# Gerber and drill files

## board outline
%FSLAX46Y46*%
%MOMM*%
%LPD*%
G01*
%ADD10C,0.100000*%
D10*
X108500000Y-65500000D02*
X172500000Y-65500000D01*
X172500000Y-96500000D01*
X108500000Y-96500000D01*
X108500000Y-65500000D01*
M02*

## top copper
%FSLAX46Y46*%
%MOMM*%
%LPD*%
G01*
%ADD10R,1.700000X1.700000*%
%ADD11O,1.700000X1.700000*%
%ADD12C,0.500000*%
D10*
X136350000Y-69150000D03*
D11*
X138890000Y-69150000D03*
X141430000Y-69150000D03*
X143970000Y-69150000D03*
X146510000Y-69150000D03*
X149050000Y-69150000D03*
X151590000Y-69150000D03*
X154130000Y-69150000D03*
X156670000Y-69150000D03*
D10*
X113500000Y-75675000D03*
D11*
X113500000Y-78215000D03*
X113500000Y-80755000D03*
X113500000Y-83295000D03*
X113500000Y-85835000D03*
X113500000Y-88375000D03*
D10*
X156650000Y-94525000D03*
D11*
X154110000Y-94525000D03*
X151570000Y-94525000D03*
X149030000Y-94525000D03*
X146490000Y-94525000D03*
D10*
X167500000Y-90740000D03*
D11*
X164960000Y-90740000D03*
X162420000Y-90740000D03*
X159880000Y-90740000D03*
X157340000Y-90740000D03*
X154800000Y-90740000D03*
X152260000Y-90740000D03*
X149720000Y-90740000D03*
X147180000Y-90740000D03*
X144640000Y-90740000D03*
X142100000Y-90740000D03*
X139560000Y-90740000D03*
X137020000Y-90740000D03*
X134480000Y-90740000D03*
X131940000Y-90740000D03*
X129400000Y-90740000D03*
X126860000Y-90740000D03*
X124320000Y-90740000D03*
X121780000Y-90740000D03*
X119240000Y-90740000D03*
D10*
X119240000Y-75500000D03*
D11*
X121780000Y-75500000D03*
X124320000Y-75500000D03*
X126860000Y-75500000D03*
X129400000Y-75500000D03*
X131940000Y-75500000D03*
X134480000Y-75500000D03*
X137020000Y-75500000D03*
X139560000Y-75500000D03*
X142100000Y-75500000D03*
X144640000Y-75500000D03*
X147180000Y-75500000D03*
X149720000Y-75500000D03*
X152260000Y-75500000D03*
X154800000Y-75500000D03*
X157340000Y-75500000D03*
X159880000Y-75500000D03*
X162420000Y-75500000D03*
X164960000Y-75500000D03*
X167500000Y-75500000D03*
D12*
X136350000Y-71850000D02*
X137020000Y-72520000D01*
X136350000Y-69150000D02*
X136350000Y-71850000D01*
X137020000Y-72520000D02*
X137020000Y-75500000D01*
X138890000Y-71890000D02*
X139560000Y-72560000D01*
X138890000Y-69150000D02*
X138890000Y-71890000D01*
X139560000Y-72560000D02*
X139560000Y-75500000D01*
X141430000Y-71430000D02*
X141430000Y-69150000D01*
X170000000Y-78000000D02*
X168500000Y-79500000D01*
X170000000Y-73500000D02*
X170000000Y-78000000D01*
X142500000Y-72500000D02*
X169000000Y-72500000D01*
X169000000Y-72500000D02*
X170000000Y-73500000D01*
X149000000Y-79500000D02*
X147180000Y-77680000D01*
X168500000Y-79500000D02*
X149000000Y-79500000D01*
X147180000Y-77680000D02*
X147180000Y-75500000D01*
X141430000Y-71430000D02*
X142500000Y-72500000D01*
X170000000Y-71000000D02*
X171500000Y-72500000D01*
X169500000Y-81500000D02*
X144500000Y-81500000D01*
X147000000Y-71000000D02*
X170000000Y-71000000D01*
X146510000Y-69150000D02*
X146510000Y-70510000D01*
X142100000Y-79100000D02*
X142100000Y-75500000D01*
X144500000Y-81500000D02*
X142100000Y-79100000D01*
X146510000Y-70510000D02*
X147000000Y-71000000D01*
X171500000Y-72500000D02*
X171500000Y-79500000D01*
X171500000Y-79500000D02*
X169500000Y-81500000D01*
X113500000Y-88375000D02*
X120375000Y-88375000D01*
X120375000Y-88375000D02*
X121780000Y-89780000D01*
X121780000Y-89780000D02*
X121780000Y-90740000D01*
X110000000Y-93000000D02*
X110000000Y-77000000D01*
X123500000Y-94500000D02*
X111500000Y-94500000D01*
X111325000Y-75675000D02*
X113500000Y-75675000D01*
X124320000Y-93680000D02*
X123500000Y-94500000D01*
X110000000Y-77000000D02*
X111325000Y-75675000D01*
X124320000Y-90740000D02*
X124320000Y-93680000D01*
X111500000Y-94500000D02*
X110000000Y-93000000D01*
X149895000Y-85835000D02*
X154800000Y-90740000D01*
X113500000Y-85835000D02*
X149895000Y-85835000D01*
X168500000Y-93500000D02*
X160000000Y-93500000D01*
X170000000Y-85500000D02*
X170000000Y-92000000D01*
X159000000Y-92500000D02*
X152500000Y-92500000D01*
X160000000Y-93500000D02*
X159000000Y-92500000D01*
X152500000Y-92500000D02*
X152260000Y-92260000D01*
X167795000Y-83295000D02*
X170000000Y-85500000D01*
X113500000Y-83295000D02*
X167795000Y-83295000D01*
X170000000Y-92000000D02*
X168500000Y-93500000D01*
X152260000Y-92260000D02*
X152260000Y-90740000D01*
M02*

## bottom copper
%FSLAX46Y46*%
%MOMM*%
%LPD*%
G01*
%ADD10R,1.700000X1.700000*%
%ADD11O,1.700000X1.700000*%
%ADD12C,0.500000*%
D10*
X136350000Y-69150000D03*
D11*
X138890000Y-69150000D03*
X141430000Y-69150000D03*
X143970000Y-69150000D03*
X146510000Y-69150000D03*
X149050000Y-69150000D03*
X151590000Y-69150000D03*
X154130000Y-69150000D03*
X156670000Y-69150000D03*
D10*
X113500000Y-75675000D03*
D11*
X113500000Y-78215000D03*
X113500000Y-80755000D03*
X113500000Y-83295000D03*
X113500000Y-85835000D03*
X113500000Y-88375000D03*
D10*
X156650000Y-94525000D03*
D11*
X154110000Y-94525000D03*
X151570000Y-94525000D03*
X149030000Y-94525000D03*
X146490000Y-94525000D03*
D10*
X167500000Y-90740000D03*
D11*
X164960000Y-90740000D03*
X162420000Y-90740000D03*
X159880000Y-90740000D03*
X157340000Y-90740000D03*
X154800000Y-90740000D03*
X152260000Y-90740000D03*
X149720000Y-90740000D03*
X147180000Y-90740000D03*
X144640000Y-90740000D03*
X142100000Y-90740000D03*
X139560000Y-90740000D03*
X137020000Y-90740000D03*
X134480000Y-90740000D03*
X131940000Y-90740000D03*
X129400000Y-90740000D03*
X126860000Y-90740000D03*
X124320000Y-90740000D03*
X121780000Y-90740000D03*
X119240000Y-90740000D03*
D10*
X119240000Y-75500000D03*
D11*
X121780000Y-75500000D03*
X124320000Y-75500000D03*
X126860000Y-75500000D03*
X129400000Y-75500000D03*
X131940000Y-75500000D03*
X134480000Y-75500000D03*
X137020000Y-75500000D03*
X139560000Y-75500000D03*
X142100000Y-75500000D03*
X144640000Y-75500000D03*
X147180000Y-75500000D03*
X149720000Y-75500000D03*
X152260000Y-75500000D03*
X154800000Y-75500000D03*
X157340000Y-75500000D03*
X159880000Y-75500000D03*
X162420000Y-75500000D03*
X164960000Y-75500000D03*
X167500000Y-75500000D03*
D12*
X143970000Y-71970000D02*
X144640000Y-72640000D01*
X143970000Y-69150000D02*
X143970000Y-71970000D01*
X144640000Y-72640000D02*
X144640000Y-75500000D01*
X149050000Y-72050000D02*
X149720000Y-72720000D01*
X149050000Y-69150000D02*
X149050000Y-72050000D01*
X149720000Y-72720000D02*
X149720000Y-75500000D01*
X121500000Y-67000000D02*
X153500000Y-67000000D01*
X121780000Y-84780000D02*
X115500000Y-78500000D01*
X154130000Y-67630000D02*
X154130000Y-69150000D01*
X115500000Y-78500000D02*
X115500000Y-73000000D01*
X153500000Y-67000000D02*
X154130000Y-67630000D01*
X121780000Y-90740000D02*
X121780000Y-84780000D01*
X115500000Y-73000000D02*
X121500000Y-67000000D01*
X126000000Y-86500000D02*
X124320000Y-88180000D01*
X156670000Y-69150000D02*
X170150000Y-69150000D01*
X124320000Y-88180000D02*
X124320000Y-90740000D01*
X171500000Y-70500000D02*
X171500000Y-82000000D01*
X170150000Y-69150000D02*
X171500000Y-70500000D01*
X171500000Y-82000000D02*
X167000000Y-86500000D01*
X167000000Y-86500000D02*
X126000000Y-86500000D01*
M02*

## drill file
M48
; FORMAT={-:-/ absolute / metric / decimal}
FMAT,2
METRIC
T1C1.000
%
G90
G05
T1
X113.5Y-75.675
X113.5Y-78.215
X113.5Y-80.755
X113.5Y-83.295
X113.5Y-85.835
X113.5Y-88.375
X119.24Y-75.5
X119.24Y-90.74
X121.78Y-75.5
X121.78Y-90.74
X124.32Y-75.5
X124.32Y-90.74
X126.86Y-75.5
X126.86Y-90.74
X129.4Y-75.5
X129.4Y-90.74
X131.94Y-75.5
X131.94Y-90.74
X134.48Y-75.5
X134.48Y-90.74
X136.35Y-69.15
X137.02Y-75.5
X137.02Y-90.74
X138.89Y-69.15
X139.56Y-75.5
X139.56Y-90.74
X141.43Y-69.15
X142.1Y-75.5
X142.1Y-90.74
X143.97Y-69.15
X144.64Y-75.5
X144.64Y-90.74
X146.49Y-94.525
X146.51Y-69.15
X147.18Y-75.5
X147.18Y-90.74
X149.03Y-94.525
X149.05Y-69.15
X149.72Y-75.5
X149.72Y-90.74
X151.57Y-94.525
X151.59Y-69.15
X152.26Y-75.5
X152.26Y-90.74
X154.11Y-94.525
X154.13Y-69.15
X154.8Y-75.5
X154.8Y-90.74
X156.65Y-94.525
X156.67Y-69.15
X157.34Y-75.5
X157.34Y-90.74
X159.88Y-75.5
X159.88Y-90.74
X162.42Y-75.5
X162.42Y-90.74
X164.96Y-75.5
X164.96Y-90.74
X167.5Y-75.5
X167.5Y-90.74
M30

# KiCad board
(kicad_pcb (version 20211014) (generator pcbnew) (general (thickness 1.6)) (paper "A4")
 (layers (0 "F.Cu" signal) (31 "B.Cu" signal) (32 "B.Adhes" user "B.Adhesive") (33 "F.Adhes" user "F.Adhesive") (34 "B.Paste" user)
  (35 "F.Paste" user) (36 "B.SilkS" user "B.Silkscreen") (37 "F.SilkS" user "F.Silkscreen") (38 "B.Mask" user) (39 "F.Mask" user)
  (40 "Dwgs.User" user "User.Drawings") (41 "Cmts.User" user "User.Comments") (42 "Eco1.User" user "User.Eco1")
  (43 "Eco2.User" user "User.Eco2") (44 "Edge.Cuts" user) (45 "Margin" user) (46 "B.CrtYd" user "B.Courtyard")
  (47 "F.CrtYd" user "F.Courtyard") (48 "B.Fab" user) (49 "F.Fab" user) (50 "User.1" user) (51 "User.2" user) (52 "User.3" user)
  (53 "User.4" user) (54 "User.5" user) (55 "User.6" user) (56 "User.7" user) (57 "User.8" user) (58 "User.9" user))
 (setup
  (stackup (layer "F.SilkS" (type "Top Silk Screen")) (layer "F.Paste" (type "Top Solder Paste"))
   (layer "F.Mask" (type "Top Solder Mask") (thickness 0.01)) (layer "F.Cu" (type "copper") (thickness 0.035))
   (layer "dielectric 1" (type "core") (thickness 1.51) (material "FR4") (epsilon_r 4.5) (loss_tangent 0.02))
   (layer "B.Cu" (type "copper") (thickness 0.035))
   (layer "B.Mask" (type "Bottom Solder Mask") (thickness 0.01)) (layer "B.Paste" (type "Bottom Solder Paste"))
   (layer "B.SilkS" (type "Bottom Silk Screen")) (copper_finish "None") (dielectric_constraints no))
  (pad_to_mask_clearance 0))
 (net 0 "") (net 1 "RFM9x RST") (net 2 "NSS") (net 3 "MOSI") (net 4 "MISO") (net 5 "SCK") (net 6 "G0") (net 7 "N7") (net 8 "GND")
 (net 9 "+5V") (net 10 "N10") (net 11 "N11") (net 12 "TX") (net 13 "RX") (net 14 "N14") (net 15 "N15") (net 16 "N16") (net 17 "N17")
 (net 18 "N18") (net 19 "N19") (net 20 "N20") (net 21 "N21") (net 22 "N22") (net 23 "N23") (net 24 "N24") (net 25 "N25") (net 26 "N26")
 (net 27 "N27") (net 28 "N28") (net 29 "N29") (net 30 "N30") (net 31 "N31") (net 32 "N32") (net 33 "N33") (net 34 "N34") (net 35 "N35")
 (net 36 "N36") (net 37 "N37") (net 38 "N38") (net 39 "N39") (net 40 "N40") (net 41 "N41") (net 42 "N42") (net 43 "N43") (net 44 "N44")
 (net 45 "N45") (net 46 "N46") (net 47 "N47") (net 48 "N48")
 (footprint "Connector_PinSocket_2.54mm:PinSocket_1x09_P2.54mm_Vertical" (layer "F.Cu") (at 136.35 69.15 90)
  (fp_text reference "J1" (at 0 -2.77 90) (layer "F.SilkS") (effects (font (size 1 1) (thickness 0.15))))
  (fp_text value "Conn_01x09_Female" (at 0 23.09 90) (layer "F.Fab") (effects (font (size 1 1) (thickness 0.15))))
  (pad "1" thru_hole rect locked (at 0 0 90) (size 1.7 1.7) (drill 1) (layers *.Cu *.Mask) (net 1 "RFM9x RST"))
  (pad "2" thru_hole oval locked (at 0 2.54 90) (size 1.7 1.7) (drill 1) (layers *.Cu *.Mask) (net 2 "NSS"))
  (pad "3" thru_hole oval locked (at 0 5.08 90) (size 1.7 1.7) (drill 1) (layers *.Cu *.Mask) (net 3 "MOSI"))
  (pad "4" thru_hole oval locked (at 0 7.62 90) (size 1.7 1.7) (drill 1) (layers *.Cu *.Mask) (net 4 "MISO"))
  (pad "5" thru_hole oval locked (at 0 10.16 90) (size 1.7 1.7) (drill 1) (layers *.Cu *.Mask) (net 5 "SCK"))
  (pad "6" thru_hole oval locked (at 0 12.7 90) (size 1.7 1.7) (drill 1) (layers *.Cu *.Mask) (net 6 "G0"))
  (pad "7" thru_hole oval locked (at 0 15.24 90) (size 1.7 1.7) (drill 1) (layers *.Cu *.Mask) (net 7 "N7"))
  (pad "8" thru_hole oval locked (at 0 17.78 90) (size 1.7 1.7) (drill 1) (layers *.Cu *.Mask) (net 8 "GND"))
  (pad "9" thru_hole oval locked (at 0 20.32 90) (size 1.7 1.7) (drill 1) (layers *.Cu *.Mask) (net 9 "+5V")))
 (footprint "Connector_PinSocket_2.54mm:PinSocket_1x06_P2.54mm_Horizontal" (layer "F.Cu") (at 113.5 75.675)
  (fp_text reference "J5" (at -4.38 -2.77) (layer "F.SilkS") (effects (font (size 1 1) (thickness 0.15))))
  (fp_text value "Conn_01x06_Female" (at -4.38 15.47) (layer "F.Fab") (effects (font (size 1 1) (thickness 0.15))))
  (pad "1" thru_hole rect locked (at 0 0) (size 1.7 1.7) (drill 1) (layers *.Cu *.Mask) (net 9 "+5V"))
  (pad "2" thru_hole oval locked (at 0 2.54) (size 1.7 1.7) (drill 1) (layers *.Cu *.Mask) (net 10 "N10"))
  (pad "3" thru_hole oval locked (at 0 5.08) (size 1.7 1.7) (drill 1) (layers *.Cu *.Mask) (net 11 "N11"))
  (pad "4" thru_hole oval locked (at 0 7.62) (size 1.7 1.7) (drill 1) (layers *.Cu *.Mask) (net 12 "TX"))
  (pad "5" thru_hole oval locked (at 0 10.16) (size 1.7 1.7) (drill 1) (layers *.Cu *.Mask) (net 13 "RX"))
  (pad "6" thru_hole oval locked (at 0 12.7) (size 1.7 1.7) (drill 1) (layers *.Cu *.Mask) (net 8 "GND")))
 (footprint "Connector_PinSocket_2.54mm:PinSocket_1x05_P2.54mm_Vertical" (layer "F.Cu") (at 156.65 94.525 -90)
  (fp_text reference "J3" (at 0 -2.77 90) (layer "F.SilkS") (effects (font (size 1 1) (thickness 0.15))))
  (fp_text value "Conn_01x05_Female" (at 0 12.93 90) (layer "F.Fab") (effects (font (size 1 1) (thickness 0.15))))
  (pad "1" thru_hole rect locked (at 0 0 270) (size 1.7 1.7) (drill 1) (layers *.Cu *.Mask) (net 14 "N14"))
  (pad "2" thru_hole oval locked (at 0 2.54 270) (size 1.7 1.7) (drill 1) (layers *.Cu *.Mask) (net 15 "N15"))
  (pad "3" thru_hole oval locked (at 0 5.08 270) (size 1.7 1.7) (drill 1) (layers *.Cu *.Mask) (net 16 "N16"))
  (pad "4" thru_hole oval locked (at 0 7.62 270) (size 1.7 1.7) (drill 1) (layers *.Cu *.Mask) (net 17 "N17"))
  (pad "5" thru_hole oval locked (at 0 10.16 270) (size 1.7 1.7) (drill 1) (layers *.Cu *.Mask) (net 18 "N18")))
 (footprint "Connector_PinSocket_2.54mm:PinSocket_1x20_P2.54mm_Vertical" (layer "B.Cu") (at 167.5 90.74 90)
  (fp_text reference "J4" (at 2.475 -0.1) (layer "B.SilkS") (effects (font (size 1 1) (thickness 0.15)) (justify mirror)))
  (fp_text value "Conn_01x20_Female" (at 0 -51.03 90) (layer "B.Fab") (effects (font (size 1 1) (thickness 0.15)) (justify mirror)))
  (pad "1" thru_hole rect locked (at 0 0 90) (size 1.7 1.7) (drill 1) (layers *.Cu *.Mask) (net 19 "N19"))
  (pad "2" thru_hole oval locked (at 0 -2.54 90) (size 1.7 1.7) (drill 1) (layers *.Cu *.Mask) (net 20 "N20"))
  (pad "3" thru_hole oval locked (at 0 -5.08 90) (size 1.7 1.7) (drill 1) (layers *.Cu *.Mask) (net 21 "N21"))
  (pad "4" thru_hole oval locked (at 0 -7.62 90) (size 1.7 1.7) (drill 1) (layers *.Cu *.Mask) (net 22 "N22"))
  (pad "5" thru_hole oval locked (at 0 -10.16 90) (size 1.7 1.7) (drill 1) (layers *.Cu *.Mask) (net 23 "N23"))
  (pad "6" thru_hole oval locked (at 0 -12.7 90) (size 1.7 1.7) (drill 1) (layers *.Cu *.Mask) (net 13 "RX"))
  (pad "7" thru_hole oval locked (at 0 -15.24 90) (size 1.7 1.7) (drill 1) (layers *.Cu *.Mask) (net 12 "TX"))
  (pad "8" thru_hole oval locked (at 0 -17.78 90) (size 1.7 1.7) (drill 1) (layers *.Cu *.Mask) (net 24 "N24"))
  (pad "9" thru_hole oval locked (at 0 -20.32 90) (size 1.7 1.7) (drill 1) (layers *.Cu *.Mask) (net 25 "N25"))
  (pad "10" thru_hole oval locked (at 0 -22.86 90) (size 1.7 1.7) (drill 1) (layers *.Cu *.Mask) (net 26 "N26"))
  (pad "11" thru_hole oval locked (at 0 -25.4 90) (size 1.7 1.7) (drill 1) (layers *.Cu *.Mask) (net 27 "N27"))
  (pad "12" thru_hole oval locked (at 0 -27.94 90) (size 1.7 1.7) (drill 1) (layers *.Cu *.Mask) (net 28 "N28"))
  (pad "13" thru_hole oval locked (at 0 -30.48 90) (size 1.7 1.7) (drill 1) (layers *.Cu *.Mask) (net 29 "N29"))
  (pad "14" thru_hole oval locked (at 0 -33.02 90) (size 1.7 1.7) (drill 1) (layers *.Cu *.Mask) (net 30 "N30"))
  (pad "15" thru_hole oval locked (at 0 -35.56 90) (size 1.7 1.7) (drill 1) (layers *.Cu *.Mask) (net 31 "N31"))
  (pad "16" thru_hole oval locked (at 0 -38.1 90) (size 1.7 1.7) (drill 1) (layers *.Cu *.Mask) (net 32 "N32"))
  (pad "17" thru_hole oval locked (at 0 -40.64 90) (size 1.7 1.7) (drill 1) (layers *.Cu *.Mask) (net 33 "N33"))
  (pad "18" thru_hole oval locked (at 0 -43.18 90) (size 1.7 1.7) (drill 1) (layers *.Cu *.Mask) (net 9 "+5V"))
  (pad "19" thru_hole oval locked (at 0 -45.72 90) (size 1.7 1.7) (drill 1) (layers *.Cu *.Mask) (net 8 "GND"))
  (pad "20" thru_hole oval locked (at 0 -48.26 90) (size 1.7 1.7) (drill 1) (layers *.Cu *.Mask) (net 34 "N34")))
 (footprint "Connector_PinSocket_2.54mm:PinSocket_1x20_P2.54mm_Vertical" (layer "B.Cu") (at 119.24 75.5 -90)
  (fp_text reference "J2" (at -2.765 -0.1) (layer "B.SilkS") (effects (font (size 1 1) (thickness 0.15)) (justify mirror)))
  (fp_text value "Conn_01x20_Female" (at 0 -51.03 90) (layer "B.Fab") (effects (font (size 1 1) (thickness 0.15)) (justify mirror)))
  (pad "1" thru_hole rect locked (at 0 0 270) (size 1.7 1.7) (drill 1) (layers *.Cu *.Mask) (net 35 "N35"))
  (pad "2" thru_hole oval locked (at 0 -2.54 270) (size 1.7 1.7) (drill 1) (layers *.Cu *.Mask) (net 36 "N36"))
  (pad "3" thru_hole oval locked (at 0 -5.08 270) (size 1.7 1.7) (drill 1) (layers *.Cu *.Mask) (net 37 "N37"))
  (pad "4" thru_hole oval locked (at 0 -7.62 270) (size 1.7 1.7) (drill 1) (layers *.Cu *.Mask) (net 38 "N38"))
  (pad "5" thru_hole oval locked (at 0 -10.16 270) (size 1.7 1.7) (drill 1) (layers *.Cu *.Mask) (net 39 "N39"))
  (pad "6" thru_hole oval locked (at 0 -12.7 270) (size 1.7 1.7) (drill 1) (layers *.Cu *.Mask) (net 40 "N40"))
  (pad "7" thru_hole oval locked (at 0 -15.24 270) (size 1.7 1.7) (drill 1) (layers *.Cu *.Mask) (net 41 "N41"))
  (pad "8" thru_hole oval locked (at 0 -17.78 270) (size 1.7 1.7) (drill 1) (layers *.Cu *.Mask) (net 1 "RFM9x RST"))
  (pad "9" thru_hole oval locked (at 0 -20.32 270) (size 1.7 1.7) (drill 1) (layers *.Cu *.Mask) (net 2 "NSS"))
  (pad "10" thru_hole oval locked (at 0 -22.86 270) (size 1.7 1.7) (drill 1) (layers *.Cu *.Mask) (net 5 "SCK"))
  (pad "11" thru_hole oval locked (at 0 -25.4 270) (size 1.7 1.7) (drill 1) (layers *.Cu *.Mask) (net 4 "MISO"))
  (pad "12" thru_hole oval locked (at 0 -27.94 270) (size 1.7 1.7) (drill 1) (layers *.Cu *.Mask) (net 3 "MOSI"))
  (pad "13" thru_hole oval locked (at 0 -30.48 270) (size 1.7 1.7) (drill 1) (layers *.Cu *.Mask) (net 6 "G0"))
  (pad "14" thru_hole oval locked (at 0 -33.02 270) (size 1.7 1.7) (drill 1) (layers *.Cu *.Mask) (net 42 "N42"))
  (pad "15" thru_hole oval locked (at 0 -35.56 270) (size 1.7 1.7) (drill 1) (layers *.Cu *.Mask) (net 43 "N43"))
  (pad "16" thru_hole oval locked (at 0 -38.1 270) (size 1.7 1.7) (drill 1) (layers *.Cu *.Mask) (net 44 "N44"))
  (pad "17" thru_hole oval locked (at 0 -40.64 270) (size 1.7 1.7) (drill 1) (layers *.Cu *.Mask) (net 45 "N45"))
  (pad "18" thru_hole oval locked (at 0 -43.18 270) (size 1.7 1.7) (drill 1) (layers *.Cu *.Mask) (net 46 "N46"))
  (pad "19" thru_hole oval locked (at 0 -45.72 270) (size 1.7 1.7) (drill 1) (layers *.Cu *.Mask) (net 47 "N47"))
  (pad "20" thru_hole oval locked (at 0 -48.26 270) (size 1.7 1.7) (drill 1) (layers *.Cu *.Mask) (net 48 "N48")))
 (gr_rect (start 108.5 65.5) (end 172.5 96.5) (layer "Edge.Cuts") (width 0.1) (fill none))
 (segment (start 136.35 71.85) (end 137.02 72.52) (width 0.5) (layer "F.Cu") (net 1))
 (segment (start 136.35 69.15) (end 136.35 71.85) (width 0.5) (layer "F.Cu") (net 1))
 (segment (start 137.02 72.52) (end 137.02 75.5) (width 0.5) (layer "F.Cu") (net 1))
 (segment (start 138.89 71.89) (end 139.56 72.56) (width 0.5) (layer "F.Cu") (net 2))
 (segment (start 138.89 69.15) (end 138.89 71.89) (width 0.5) (layer "F.Cu") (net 2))
 (segment (start 139.56 72.56) (end 139.56 75.5) (width 0.5) (layer "F.Cu") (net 2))
 (segment (start 141.43 71.43) (end 141.43 69.15) (width 0.5) (layer "F.Cu") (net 3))
 (segment (start 170 78) (end 168.5 79.5) (width 0.5) (layer "F.Cu") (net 3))
 (segment (start 170 73.5) (end 170 78) (width 0.5) (layer "F.Cu") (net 3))
 (segment (start 142.5 72.5) (end 169 72.5) (width 0.5) (layer "F.Cu") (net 3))
 (segment (start 169 72.5) (end 170 73.5) (width 0.5) (layer "F.Cu") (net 3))
 (segment (start 149 79.5) (end 147.18 77.68) (width 0.5) (layer "F.Cu") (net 3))
 (segment (start 168.5 79.5) (end 149 79.5) (width 0.5) (layer "F.Cu") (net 3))
 (segment (start 147.18 77.68) (end 147.18 75.5) (width 0.5) (layer "F.Cu") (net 3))
 (segment (start 141.43 71.43) (end 142.5 72.5) (width 0.5) (layer "F.Cu") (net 3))
 (segment (start 143.97 71.97) (end 144.64 72.64) (width 0.5) (layer "B.Cu") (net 4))
 (segment (start 143.97 69.15) (end 143.97 71.97) (width 0.5) (layer "B.Cu") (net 4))
 (segment (start 144.64 72.64) (end 144.64 75.5) (width 0.5) (layer "B.Cu") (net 4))
 (segment (start 170 71) (end 171.5 72.5) (width 0.5) (layer "F.Cu") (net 5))
 (segment (start 169.5 81.5) (end 144.5 81.5) (width 0.5) (layer "F.Cu") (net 5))
 (segment (start 147 71) (end 170 71) (width 0.5) (layer "F.Cu") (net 5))
 (segment (start 146.51 69.15) (end 146.51 70.51) (width 0.5) (layer "F.Cu") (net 5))
 (segment (start 142.1 79.1) (end 142.1 75.5) (width 0.5) (layer "F.Cu") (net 5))
 (segment (start 144.5 81.5) (end 142.1 79.1) (width 0.5) (layer "F.Cu") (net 5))
 (segment (start 146.51 70.51) (end 147 71) (width 0.5) (layer "F.Cu") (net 5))
 (segment (start 171.5 72.5) (end 171.5 79.5) (width 0.5) (layer "F.Cu") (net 5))
 (segment (start 171.5 79.5) (end 169.5 81.5) (width 0.5) (layer "F.Cu") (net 5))
 (segment (start 149.05 72.05) (end 149.72 72.72) (width 0.5) (layer "B.Cu") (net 6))
 (segment (start 149.05 69.15) (end 149.05 72.05) (width 0.5) (layer "B.Cu") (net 6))
 (segment (start 149.72 72.72) (end 149.72 75.5) (width 0.5) (layer "B.Cu") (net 6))
 (segment (start 113.5 88.375) (end 120.375 88.375) (width 0.5) (layer "F.Cu") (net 8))
 (segment (start 120.375 88.375) (end 121.78 89.78) (width 0.5) (layer "F.Cu") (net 8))
 (segment (start 121.78 89.78) (end 121.78 90.74) (width 0.5) (layer "F.Cu") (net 8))
 (segment (start 121.5 67) (end 153.5 67) (width 0.5) (layer "B.Cu") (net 8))
 (segment (start 121.78 84.78) (end 115.5 78.5) (width 0.5) (layer "B.Cu") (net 8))
 (segment (start 154.13 67.63) (end 154.13 69.15) (width 0.5) (layer "B.Cu") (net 8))
 (segment (start 115.5 78.5) (end 115.5 73) (width 0.5) (layer "B.Cu") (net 8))
 (segment (start 153.5 67) (end 154.13 67.63) (width 0.5) (layer "B.Cu") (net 8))
 (segment (start 121.78 90.74) (end 121.78 84.78) (width 0.5) (layer "B.Cu") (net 8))
 (segment (start 115.5 73) (end 121.5 67) (width 0.5) (layer "B.Cu") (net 8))
 (segment (start 110 93) (end 110 77) (width 0.5) (layer "F.Cu") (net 9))
 (segment (start 123.5 94.5) (end 111.5 94.5) (width 0.5) (layer "F.Cu") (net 9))
 (segment (start 111.325 75.675) (end 113.5 75.675) (width 0.5) (layer "F.Cu") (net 9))
 (segment (start 124.32 93.68) (end 123.5 94.5) (width 0.5) (layer "F.Cu") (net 9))
 (segment (start 110 77) (end 111.325 75.675) (width 0.5) (layer "F.Cu") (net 9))
 (segment (start 124.32 90.74) (end 124.32 93.68) (width 0.5) (layer "F.Cu") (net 9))
 (segment (start 111.5 94.5) (end 110 93) (width 0.5) (layer "F.Cu") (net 9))
 (segment (start 126 86.5) (end 124.32 88.18) (width 0.5) (layer "B.Cu") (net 9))
 (segment (start 156.67 69.15) (end 170.15 69.15) (width 0.5) (layer "B.Cu") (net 9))
 (segment (start 124.32 88.18) (end 124.32 90.74) (width 0.5) (layer "B.Cu") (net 9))
 (segment (start 171.5 70.5) (end 171.5 82) (width 0.5) (layer "B.Cu") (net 9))
 (segment (start 170.15 69.15) (end 171.5 70.5) (width 0.5) (layer "B.Cu") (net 9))
 (segment (start 171.5 82) (end 167 86.5) (width 0.5) (layer "B.Cu") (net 9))
 (segment (start 167 86.5) (end 126 86.5) (width 0.5) (layer "B.Cu") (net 9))
 (segment (start 149.895 85.835) (end 154.8 90.74) (width 0.5) (layer "F.Cu") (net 13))
 (segment (start 113.5 85.835) (end 149.895 85.835) (width 0.5) (layer "F.Cu") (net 13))
 (segment (start 168.5 93.5) (end 160 93.5) (width 0.5) (layer "F.Cu") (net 12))
 (segment (start 170 85.5) (end 170 92) (width 0.5) (layer "F.Cu") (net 12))
 (segment (start 159 92.5) (end 152.5 92.5) (width 0.5) (layer "F.Cu") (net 12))
 (segment (start 160 93.5) (end 159 92.5) (width 0.5) (layer "F.Cu") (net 12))
 (segment (start 152.5 92.5) (end 152.26 92.26) (width 0.5) (layer "F.Cu") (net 12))
 (segment (start 167.795 83.295) (end 170 85.5) (width 0.5) (layer "F.Cu") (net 12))
 (segment (start 113.5 83.295) (end 167.795 83.295) (width 0.5) (layer "F.Cu") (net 12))
 (segment (start 170 92) (end 168.5 93.5) (width 0.5) (layer "F.Cu") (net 12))
 (segment (start 152.26 92.26) (end 152.26 90.74) (width 0.5) (layer "F.Cu") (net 12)))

